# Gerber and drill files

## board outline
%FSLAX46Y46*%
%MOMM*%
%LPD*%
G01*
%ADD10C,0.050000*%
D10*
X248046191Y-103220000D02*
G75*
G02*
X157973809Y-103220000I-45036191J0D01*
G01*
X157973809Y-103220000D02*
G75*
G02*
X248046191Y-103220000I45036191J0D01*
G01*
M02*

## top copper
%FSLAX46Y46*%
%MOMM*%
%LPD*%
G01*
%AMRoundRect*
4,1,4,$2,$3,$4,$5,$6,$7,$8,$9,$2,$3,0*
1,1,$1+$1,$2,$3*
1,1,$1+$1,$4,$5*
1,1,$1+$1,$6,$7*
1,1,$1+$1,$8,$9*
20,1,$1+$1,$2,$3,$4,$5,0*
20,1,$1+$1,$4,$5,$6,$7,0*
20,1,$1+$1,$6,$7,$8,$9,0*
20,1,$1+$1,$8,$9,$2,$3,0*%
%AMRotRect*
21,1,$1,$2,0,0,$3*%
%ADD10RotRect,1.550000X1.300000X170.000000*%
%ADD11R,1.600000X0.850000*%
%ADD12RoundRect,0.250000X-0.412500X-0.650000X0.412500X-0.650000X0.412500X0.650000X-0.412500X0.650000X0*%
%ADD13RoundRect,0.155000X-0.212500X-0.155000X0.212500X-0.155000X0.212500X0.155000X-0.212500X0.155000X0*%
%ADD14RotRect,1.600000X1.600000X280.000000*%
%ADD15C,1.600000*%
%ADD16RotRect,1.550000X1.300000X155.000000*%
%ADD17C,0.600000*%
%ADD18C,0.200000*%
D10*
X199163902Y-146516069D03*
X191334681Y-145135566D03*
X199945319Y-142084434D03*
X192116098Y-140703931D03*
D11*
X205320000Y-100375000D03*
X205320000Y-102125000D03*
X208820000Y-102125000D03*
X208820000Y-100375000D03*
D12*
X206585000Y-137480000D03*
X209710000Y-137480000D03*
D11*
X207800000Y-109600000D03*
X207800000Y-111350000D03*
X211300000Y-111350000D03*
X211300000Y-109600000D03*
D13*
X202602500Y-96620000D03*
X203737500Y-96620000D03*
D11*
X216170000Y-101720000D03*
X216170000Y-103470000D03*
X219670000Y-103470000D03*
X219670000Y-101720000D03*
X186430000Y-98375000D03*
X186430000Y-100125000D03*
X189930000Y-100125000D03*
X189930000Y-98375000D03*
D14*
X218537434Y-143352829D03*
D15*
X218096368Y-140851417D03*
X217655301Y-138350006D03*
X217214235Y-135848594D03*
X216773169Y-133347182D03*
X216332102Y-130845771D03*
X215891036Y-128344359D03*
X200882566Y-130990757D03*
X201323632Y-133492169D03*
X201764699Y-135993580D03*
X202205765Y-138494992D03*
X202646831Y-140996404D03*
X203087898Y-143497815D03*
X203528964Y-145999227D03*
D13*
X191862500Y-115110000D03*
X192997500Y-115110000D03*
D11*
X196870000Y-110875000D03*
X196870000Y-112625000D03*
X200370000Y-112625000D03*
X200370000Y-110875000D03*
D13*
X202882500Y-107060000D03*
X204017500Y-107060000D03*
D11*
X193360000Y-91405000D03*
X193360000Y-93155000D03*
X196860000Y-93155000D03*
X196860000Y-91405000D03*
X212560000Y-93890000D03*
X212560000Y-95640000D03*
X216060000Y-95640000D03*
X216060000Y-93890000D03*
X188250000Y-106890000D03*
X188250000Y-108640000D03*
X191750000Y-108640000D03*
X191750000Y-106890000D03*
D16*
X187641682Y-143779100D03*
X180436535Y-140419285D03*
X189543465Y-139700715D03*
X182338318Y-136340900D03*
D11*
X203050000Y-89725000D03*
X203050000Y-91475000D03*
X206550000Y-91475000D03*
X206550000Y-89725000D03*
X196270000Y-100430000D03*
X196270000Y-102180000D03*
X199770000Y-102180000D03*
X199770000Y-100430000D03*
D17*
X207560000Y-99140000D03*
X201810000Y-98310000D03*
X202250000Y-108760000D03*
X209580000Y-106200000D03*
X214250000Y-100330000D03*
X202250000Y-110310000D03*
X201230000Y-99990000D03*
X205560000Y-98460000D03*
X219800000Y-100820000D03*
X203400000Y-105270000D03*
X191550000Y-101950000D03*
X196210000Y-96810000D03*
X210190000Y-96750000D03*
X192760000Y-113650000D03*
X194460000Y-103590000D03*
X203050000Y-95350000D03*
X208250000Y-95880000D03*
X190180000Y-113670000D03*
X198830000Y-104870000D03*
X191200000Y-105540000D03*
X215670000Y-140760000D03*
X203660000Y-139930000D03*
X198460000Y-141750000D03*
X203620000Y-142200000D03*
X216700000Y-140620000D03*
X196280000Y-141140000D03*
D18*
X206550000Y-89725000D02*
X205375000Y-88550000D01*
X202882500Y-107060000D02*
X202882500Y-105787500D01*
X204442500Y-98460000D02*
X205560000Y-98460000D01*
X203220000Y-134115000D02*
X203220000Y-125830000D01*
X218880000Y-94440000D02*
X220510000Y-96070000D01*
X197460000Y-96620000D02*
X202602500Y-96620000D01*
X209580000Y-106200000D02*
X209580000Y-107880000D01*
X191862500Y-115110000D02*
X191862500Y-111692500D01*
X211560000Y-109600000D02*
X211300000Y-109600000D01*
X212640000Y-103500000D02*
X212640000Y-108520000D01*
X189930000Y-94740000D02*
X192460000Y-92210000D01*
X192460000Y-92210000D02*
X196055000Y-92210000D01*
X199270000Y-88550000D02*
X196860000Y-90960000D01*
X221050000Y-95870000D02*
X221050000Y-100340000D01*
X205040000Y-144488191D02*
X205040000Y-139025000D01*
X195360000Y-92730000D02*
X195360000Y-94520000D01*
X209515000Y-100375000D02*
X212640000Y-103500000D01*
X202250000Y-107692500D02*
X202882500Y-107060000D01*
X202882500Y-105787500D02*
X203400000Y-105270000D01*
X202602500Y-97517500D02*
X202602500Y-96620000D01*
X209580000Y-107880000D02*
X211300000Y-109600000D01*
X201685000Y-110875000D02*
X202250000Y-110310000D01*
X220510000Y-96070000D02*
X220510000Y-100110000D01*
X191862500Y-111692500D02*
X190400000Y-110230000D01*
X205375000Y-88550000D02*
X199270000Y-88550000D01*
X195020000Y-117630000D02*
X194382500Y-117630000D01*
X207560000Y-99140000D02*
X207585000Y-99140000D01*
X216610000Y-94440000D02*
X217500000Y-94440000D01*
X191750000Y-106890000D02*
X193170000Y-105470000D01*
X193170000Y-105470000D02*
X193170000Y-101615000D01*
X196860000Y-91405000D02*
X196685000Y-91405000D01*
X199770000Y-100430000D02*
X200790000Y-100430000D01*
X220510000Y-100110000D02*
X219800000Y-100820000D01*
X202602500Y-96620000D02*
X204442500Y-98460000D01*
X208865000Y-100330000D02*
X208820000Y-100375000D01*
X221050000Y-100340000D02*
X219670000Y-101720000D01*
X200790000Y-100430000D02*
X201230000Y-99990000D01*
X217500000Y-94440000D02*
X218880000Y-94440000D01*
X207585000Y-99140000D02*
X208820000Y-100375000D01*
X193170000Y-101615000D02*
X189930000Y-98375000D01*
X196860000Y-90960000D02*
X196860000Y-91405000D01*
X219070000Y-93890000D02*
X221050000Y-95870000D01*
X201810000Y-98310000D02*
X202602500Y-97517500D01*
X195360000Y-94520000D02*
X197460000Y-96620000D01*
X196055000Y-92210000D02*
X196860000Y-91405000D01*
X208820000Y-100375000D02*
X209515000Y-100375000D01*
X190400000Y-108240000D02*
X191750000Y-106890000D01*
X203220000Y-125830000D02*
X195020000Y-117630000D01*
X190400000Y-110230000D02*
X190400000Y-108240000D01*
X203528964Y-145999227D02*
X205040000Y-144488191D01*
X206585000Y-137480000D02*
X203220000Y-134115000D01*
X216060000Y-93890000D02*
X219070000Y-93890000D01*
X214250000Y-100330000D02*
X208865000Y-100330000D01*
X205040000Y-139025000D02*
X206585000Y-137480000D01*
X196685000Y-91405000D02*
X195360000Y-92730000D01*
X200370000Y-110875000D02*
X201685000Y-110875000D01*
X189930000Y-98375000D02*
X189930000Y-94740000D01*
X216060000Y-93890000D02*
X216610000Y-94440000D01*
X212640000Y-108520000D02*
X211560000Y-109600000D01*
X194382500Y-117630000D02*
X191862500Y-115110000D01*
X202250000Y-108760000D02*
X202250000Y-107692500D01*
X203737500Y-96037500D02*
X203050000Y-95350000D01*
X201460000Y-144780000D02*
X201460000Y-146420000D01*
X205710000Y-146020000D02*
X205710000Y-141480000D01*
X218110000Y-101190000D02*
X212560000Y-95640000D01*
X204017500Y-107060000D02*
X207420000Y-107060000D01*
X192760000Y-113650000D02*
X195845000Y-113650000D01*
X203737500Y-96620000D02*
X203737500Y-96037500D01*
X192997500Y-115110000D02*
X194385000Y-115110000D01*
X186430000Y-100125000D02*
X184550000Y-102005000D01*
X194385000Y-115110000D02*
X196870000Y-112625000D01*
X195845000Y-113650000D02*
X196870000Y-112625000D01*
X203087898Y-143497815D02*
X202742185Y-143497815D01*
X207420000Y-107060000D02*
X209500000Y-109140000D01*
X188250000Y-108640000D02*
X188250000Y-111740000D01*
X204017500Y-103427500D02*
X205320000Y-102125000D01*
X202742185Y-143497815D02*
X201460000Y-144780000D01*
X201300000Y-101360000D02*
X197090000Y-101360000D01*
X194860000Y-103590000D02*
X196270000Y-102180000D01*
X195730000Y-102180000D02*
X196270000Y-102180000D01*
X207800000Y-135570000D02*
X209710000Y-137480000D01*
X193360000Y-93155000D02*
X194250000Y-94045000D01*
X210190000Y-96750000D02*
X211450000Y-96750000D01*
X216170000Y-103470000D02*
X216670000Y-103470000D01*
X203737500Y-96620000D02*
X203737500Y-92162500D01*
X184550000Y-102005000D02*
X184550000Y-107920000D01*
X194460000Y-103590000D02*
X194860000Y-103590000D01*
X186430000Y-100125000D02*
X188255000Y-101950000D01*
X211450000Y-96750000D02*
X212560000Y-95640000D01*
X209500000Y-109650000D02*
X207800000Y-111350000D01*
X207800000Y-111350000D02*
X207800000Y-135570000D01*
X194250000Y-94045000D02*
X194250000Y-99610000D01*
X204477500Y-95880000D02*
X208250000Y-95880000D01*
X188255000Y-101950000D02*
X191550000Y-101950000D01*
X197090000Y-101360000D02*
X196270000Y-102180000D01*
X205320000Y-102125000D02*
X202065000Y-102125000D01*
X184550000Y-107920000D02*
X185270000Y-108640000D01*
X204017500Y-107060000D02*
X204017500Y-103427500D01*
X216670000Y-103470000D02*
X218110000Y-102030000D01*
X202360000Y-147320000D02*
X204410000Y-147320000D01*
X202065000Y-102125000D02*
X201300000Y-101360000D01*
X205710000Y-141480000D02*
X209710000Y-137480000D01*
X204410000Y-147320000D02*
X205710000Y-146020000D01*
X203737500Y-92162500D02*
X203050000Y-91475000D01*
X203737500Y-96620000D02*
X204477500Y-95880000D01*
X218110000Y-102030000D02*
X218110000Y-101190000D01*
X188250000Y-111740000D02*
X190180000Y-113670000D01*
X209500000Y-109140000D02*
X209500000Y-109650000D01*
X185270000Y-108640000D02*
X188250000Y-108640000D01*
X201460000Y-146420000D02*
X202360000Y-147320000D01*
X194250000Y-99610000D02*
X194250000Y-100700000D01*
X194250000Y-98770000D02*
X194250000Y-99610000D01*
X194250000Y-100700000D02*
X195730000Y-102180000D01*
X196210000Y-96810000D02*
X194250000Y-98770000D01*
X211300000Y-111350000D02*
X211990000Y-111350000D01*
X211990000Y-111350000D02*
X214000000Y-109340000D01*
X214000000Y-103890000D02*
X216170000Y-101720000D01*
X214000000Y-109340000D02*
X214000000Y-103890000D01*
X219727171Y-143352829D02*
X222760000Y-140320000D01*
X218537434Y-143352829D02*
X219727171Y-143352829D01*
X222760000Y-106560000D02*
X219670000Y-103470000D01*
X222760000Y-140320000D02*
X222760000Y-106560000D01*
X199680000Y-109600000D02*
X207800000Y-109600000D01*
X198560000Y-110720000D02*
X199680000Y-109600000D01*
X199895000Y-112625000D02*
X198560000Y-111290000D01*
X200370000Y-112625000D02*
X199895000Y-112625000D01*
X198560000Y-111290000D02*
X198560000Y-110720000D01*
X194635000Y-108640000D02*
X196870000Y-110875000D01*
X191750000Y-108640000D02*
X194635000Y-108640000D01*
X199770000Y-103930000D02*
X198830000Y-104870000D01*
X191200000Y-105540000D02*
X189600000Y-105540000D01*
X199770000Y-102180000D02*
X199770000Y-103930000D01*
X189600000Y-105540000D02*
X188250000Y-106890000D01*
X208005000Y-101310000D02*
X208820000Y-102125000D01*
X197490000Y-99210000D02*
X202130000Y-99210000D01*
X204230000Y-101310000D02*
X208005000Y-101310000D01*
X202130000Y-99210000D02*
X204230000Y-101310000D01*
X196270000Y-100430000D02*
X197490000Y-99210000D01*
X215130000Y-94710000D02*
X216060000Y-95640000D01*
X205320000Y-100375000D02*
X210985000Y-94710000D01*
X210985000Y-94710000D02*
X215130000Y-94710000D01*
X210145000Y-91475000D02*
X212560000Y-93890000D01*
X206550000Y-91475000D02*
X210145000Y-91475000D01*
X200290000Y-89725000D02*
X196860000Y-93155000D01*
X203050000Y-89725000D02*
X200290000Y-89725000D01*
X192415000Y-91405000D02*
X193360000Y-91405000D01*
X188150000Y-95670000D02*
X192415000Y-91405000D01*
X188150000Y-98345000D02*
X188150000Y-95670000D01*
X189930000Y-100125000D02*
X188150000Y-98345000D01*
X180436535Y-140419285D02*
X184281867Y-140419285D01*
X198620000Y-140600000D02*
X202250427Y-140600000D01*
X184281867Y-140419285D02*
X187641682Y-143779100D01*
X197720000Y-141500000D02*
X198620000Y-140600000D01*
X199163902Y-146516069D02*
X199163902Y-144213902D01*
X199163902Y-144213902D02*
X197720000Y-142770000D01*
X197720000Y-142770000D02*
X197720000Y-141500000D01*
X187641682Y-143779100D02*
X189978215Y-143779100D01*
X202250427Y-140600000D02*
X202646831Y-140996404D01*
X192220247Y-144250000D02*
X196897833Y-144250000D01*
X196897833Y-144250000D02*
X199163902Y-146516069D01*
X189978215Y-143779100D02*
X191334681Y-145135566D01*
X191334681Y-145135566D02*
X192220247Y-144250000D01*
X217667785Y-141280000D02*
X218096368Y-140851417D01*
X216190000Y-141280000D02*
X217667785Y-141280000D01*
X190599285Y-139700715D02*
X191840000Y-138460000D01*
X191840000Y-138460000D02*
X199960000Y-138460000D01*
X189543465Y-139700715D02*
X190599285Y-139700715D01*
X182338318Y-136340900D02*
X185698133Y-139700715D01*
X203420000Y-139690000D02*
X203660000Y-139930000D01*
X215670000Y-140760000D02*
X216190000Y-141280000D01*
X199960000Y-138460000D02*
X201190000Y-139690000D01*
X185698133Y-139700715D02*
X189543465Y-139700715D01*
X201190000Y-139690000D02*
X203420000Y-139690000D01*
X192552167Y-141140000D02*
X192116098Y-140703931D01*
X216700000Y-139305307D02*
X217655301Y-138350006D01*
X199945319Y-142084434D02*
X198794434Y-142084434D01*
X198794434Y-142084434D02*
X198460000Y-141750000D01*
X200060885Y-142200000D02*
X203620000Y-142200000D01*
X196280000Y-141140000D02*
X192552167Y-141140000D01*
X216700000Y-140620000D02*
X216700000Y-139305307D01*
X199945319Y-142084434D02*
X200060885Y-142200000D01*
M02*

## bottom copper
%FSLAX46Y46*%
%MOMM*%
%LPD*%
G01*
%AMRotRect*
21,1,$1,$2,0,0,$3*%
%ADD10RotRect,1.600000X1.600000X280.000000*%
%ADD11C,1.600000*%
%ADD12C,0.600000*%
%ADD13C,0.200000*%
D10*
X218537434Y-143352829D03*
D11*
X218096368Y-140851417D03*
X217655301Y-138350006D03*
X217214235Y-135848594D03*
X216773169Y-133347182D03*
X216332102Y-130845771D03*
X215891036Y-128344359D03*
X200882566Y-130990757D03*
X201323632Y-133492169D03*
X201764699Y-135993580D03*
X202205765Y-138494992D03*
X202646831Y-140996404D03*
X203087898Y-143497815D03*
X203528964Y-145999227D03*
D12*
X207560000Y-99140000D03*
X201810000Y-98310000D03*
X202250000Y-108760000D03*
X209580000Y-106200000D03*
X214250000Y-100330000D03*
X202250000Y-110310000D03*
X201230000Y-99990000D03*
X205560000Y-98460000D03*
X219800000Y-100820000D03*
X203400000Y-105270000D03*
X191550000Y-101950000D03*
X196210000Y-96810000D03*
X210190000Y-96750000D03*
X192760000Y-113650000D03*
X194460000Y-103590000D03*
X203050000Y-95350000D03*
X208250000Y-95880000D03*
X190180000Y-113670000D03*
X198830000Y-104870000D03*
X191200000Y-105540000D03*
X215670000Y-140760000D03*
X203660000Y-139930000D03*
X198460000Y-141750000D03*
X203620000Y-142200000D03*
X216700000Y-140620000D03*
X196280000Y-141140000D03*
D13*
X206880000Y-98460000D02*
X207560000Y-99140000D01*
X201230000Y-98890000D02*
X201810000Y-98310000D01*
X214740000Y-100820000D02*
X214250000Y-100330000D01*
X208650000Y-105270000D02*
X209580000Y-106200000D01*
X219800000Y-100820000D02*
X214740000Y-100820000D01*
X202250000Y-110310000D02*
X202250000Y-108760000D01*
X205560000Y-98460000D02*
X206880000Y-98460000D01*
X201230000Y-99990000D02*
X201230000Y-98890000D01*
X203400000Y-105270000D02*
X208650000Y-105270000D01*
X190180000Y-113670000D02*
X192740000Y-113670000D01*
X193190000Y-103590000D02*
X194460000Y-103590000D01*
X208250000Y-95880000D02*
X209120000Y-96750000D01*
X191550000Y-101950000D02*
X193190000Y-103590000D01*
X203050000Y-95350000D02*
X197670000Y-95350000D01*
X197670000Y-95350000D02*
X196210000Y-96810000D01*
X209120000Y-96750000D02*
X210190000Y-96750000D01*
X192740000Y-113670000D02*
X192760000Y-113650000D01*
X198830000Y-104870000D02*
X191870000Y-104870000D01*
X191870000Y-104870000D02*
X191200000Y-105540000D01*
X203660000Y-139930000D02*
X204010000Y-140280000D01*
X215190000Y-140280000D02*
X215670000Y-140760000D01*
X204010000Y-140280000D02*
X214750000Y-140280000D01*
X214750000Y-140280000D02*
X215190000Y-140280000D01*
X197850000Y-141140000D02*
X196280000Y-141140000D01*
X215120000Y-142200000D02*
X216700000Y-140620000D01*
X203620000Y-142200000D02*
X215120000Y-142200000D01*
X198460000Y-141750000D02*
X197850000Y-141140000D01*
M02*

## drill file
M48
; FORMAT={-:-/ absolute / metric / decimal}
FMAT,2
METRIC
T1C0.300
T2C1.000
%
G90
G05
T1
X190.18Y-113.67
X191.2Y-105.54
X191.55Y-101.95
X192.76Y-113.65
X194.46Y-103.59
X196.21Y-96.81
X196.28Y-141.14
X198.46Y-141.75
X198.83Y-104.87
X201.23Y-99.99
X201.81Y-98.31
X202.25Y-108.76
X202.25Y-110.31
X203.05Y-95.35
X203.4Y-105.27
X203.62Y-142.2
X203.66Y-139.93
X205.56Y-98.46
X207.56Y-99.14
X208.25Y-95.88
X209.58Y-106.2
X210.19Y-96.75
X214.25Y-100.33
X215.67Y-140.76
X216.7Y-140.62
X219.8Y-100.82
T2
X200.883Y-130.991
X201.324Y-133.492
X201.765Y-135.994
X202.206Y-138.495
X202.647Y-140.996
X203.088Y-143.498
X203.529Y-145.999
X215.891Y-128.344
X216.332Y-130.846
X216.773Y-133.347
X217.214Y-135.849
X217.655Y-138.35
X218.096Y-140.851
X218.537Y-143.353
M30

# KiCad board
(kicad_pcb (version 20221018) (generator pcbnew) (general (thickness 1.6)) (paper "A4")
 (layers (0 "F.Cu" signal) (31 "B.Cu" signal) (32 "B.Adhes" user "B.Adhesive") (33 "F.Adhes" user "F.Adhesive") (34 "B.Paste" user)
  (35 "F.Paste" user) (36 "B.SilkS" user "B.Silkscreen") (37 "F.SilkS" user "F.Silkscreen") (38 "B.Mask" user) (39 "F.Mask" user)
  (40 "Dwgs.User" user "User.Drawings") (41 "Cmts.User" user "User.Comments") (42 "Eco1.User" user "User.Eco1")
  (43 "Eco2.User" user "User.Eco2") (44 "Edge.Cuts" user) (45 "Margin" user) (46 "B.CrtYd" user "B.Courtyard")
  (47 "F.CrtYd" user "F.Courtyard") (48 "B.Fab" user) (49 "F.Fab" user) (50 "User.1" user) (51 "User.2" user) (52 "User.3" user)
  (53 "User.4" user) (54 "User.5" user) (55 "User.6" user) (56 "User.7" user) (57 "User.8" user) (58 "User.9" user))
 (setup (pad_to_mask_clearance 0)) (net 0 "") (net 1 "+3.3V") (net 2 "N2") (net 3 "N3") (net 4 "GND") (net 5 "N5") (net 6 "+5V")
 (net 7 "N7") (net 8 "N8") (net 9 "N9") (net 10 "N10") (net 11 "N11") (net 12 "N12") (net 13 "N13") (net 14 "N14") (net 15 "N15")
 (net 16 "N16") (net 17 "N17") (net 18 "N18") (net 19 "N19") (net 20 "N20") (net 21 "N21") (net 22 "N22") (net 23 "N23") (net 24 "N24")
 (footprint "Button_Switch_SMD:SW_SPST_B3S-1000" (layer "F.Cu") (at 195.64 143.61 170)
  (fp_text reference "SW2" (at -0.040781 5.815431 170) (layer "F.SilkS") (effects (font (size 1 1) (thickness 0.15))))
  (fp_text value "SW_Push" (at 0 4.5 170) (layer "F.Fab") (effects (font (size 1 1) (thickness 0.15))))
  (pad "1" smd rect (at -3.975 -2.25 170) (size 1.55 1.3) (layers "F.Cu" "F.Paste" "F.Mask") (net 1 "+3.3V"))
  (pad "1" smd rect (at 3.975 -2.25 170) (size 1.55 1.3) (layers "F.Cu" "F.Paste" "F.Mask") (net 1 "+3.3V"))
  (pad "2" smd rect (at -3.975 2.25 170) (size 1.55 1.3) (layers "F.Cu" "F.Paste" "F.Mask") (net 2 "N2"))
  (pad "2" smd rect (at 3.975 2.25 170) (size 1.55 1.3) (layers "F.Cu" "F.Paste" "F.Mask") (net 2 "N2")))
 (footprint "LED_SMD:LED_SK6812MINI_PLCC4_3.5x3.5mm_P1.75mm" (layer "F.Cu") (at 207.07 101.25)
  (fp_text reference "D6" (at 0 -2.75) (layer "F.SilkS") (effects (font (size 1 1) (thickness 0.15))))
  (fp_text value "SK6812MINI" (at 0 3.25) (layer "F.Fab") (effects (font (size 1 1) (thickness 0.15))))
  (pad "1" smd rect (at -1.75 -0.875) (size 1.6 0.85) (layers "F.Cu" "F.Paste" "F.Mask") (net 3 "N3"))
  (pad "2" smd rect (at -1.75 0.875) (size 1.6 0.85) (layers "F.Cu" "F.Paste" "F.Mask") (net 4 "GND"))
  (pad "3" smd rect (at 1.75 0.875) (size 1.6 0.85) (layers "F.Cu" "F.Paste" "F.Mask") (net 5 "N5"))
  (pad "4" smd rect (at 1.75 -0.875) (size 1.6 0.85) (layers "F.Cu" "F.Paste" "F.Mask") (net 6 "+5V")))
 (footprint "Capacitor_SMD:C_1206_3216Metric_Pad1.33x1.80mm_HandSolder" (layer "F.Cu") (at 208.1475 137.48)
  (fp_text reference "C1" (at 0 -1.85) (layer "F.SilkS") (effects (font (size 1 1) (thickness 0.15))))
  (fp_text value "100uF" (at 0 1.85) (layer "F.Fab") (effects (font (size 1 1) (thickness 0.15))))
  (pad "1" smd roundrect (at -1.5625 0) (size 1.325 1.8) (layers "F.Cu" "F.Paste" "F.Mask") (roundrect_rratio 0.1886792453) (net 6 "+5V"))
  (pad "2" smd roundrect (at 1.5625 0) (size 1.325 1.8) (layers "F.Cu" "F.Paste" "F.Mask") (roundrect_rratio 0.1886792453) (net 4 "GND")))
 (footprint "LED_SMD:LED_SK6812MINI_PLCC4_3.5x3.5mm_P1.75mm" (layer "F.Cu") (at 209.55 110.475)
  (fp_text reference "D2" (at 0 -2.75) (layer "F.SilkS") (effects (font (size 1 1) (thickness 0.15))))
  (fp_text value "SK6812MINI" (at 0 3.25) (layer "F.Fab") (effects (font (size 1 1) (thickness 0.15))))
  (pad "1" smd rect (at -1.75 -0.875) (size 1.6 0.85) (layers "F.Cu" "F.Paste" "F.Mask") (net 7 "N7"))
  (pad "2" smd rect (at -1.75 0.875) (size 1.6 0.85) (layers "F.Cu" "F.Paste" "F.Mask") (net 4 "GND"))
  (pad "3" smd rect (at 1.75 0.875) (size 1.6 0.85) (layers "F.Cu" "F.Paste" "F.Mask") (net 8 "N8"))
  (pad "4" smd rect (at 1.75 -0.875) (size 1.6 0.85) (layers "F.Cu" "F.Paste" "F.Mask") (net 6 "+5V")))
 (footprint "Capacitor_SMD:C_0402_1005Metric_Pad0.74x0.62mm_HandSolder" (layer "F.Cu") (at 203.17 96.62)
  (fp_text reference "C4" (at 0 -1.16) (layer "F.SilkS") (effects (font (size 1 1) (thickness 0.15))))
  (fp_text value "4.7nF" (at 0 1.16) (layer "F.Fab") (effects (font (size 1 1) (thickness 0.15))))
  (pad "1" smd roundrect (at -0.5675 0) (size 0.735 0.62) (layers "F.Cu" "F.Paste" "F.Mask") (roundrect_rratio 0.25) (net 6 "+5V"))
  (pad "2" smd roundrect (at 0.5675 0) (size 0.735 0.62) (layers "F.Cu" "F.Paste" "F.Mask") (roundrect_rratio 0.25) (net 4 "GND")))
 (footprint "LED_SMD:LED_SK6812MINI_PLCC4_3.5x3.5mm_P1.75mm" (layer "F.Cu") (at 217.92 102.595)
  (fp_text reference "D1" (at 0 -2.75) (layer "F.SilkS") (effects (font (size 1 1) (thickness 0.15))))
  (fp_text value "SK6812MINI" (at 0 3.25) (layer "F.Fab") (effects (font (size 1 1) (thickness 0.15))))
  (pad "1" smd rect (at -1.75 -0.875) (size 1.6 0.85) (layers "F.Cu" "F.Paste" "F.Mask") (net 8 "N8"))
  (pad "2" smd rect (at -1.75 0.875) (size 1.6 0.85) (layers "F.Cu" "F.Paste" "F.Mask") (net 4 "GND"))
  (pad "3" smd rect (at 1.75 0.875) (size 1.6 0.85) (layers "F.Cu" "F.Paste" "F.Mask") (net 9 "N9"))
  (pad "4" smd rect (at 1.75 -0.875) (size 1.6 0.85) (layers "F.Cu" "F.Paste" "F.Mask") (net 6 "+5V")))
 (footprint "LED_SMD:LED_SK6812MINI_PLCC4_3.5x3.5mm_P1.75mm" (layer "F.Cu") (at 188.18 99.25)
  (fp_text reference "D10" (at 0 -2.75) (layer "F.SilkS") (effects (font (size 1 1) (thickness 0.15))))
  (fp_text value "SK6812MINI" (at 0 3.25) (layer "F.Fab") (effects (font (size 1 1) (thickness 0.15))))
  (pad "1" smd rect (at -1.75 -0.875) (size 1.6 0.85) (layers "F.Cu" "F.Paste" "F.Mask") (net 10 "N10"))
  (pad "2" smd rect (at -1.75 0.875) (size 1.6 0.85) (layers "F.Cu" "F.Paste" "F.Mask") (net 4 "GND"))
  (pad "3" smd rect (at 1.75 0.875) (size 1.6 0.85) (layers "F.Cu" "F.Paste" "F.Mask") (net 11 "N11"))
  (pad "4" smd rect (at 1.75 -0.875) (size 1.6 0.85) (layers "F.Cu" "F.Paste" "F.Mask") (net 6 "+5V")))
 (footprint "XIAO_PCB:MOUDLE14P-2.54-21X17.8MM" (layer "F.Cu") (at 209.71 137.171793 -80)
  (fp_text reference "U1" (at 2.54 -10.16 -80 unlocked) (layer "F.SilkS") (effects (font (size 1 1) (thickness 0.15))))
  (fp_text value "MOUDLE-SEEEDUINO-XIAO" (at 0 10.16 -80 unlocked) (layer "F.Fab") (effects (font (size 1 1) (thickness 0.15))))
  (pad "1" thru_hole rect (at 7.62 -7.62 280) (size 1.6 1.6) (drill 1) (layers "*.Cu" "*.Mask") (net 9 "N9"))
  (pad "2" thru_hole circle (at 5.08 -7.62 280) (size 1.6 1.6) (drill 1) (layers "*.Cu" "*.Mask") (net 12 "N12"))
  (pad "3" thru_hole circle (at 2.54 -7.62 280) (size 1.6 1.6) (drill 1) (layers "*.Cu" "*.Mask") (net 2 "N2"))
  (pad "4" thru_hole circle (at 0 -7.62 280) (size 1.6 1.6) (drill 1) (layers "*.Cu" "*.Mask") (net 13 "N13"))
  (pad "5" thru_hole circle (at -2.54 -7.62 280) (size 1.6 1.6) (drill 1) (layers "*.Cu" "*.Mask") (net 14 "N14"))
  (pad "6" thru_hole circle (at -5.08 -7.62 280) (size 1.6 1.6) (drill 1) (layers "*.Cu" "*.Mask") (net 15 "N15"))
  (pad "7" thru_hole circle (at -7.62 -7.62 280) (size 1.6 1.6) (drill 1) (layers "*.Cu" "*.Mask") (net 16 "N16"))
  (pad "8" thru_hole circle (at -7.62 7.62 280) (size 1.6 1.6) (drill 1) (layers "*.Cu" "*.Mask") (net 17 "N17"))
  (pad "9" thru_hole circle (at -5.08 7.62 280) (size 1.6 1.6) (drill 1) (layers "*.Cu" "*.Mask") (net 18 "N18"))
  (pad "10" thru_hole circle (at -2.54 7.62 280) (size 1.6 1.6) (drill 1) (layers "*.Cu" "*.Mask") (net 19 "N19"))
  (pad "11" thru_hole circle (at 0 7.62 280) (size 1.6 1.6) (drill 1) (layers "*.Cu" "*.Mask") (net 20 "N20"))
  (pad "12" thru_hole circle (at 2.54 7.62 280) (size 1.6 1.6) (drill 1) (layers "*.Cu" "*.Mask") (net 1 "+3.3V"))
  (pad "13" thru_hole circle (at 5.08 7.62 280) (size 1.6 1.6) (drill 1) (layers "*.Cu" "*.Mask") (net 4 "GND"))
  (pad "14" thru_hole circle (at 7.62 7.62 280) (size 1.6 1.6) (drill 1) (layers "*.Cu" "*.Mask") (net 6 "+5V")))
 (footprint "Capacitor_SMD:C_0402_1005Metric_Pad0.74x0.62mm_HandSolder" (layer "F.Cu") (at 192.43 115.11)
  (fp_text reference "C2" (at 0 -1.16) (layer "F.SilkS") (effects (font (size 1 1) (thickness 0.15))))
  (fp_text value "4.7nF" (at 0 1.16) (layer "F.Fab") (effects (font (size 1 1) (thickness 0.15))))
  (pad "1" smd roundrect (at -0.5675 0) (size 0.735 0.62) (layers "F.Cu" "F.Paste" "F.Mask") (roundrect_rratio 0.25) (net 6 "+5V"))
  (pad "2" smd roundrect (at 0.5675 0) (size 0.735 0.62) (layers "F.Cu" "F.Paste" "F.Mask") (roundrect_rratio 0.25) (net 4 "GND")))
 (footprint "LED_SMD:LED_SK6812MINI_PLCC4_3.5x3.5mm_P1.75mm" (layer "F.Cu") (at 198.62 111.75)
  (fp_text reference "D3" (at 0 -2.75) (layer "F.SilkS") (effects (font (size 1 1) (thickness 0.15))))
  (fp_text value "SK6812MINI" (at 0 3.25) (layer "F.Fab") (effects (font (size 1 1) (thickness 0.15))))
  (pad "1" smd rect (at -1.75 -0.875) (size 1.6 0.85) (layers "F.Cu" "F.Paste" "F.Mask") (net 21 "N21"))
  (pad "2" smd rect (at -1.75 0.875) (size 1.6 0.85) (layers "F.Cu" "F.Paste" "F.Mask") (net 4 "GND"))
  (pad "3" smd rect (at 1.75 0.875) (size 1.6 0.85) (layers "F.Cu" "F.Paste" "F.Mask") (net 7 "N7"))
  (pad "4" smd rect (at 1.75 -0.875) (size 1.6 0.85) (layers "F.Cu" "F.Paste" "F.Mask") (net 6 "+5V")))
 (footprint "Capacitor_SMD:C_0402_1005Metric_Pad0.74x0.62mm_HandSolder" (layer "F.Cu") (at 203.45 107.06)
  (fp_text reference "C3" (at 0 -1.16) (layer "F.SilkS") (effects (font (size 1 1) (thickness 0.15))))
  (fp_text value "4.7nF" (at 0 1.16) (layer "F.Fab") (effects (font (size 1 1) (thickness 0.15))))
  (pad "1" smd roundrect (at -0.5675 0) (size 0.735 0.62) (layers "F.Cu" "F.Paste" "F.Mask") (roundrect_rratio 0.25) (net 6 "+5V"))
  (pad "2" smd roundrect (at 0.5675 0) (size 0.735 0.62) (layers "F.Cu" "F.Paste" "F.Mask") (roundrect_rratio 0.25) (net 4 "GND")))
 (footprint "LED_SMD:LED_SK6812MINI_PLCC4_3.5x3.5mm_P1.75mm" (layer "F.Cu") (at 195.11 92.28)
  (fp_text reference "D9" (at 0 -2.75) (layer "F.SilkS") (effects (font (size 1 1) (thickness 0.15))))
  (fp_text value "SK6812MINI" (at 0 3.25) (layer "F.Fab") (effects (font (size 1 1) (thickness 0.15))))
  (pad "1" smd rect (at -1.75 -0.875) (size 1.6 0.85) (layers "F.Cu" "F.Paste" "F.Mask") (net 11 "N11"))
  (pad "2" smd rect (at -1.75 0.875) (size 1.6 0.85) (layers "F.Cu" "F.Paste" "F.Mask") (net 4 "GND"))
  (pad "3" smd rect (at 1.75 0.875) (size 1.6 0.85) (layers "F.Cu" "F.Paste" "F.Mask") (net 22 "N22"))
  (pad "4" smd rect (at 1.75 -0.875) (size 1.6 0.85) (layers "F.Cu" "F.Paste" "F.Mask") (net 6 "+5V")))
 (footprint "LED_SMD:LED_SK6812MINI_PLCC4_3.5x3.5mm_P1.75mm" (layer "F.Cu") (at 214.31 94.765)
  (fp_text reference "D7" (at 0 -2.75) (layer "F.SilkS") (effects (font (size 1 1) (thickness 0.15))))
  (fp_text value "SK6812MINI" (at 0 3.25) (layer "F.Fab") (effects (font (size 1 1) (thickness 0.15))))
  (pad "1" smd rect (at -1.75 -0.875) (size 1.6 0.85) (layers "F.Cu" "F.Paste" "F.Mask") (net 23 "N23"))
  (pad "2" smd rect (at -1.75 0.875) (size 1.6 0.85) (layers "F.Cu" "F.Paste" "F.Mask") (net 4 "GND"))
  (pad "3" smd rect (at 1.75 0.875) (size 1.6 0.85) (layers "F.Cu" "F.Paste" "F.Mask") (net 3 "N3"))
  (pad "4" smd rect (at 1.75 -0.875) (size 1.6 0.85) (layers "F.Cu" "F.Paste" "F.Mask") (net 6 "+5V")))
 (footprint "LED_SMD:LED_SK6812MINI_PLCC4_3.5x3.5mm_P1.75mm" (layer "F.Cu") (at 190 107.765)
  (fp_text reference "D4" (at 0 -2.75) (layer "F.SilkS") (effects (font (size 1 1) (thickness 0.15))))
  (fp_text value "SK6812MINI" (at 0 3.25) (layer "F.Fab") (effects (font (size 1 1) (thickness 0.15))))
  (pad "1" smd rect (at -1.75 -0.875) (size 1.6 0.85) (layers "F.Cu" "F.Paste" "F.Mask") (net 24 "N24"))
  (pad "2" smd rect (at -1.75 0.875) (size 1.6 0.85) (layers "F.Cu" "F.Paste" "F.Mask") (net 4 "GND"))
  (pad "3" smd rect (at 1.75 0.875) (size 1.6 0.85) (layers "F.Cu" "F.Paste" "F.Mask") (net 21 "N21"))
  (pad "4" smd rect (at 1.75 -0.875) (size 1.6 0.85) (layers "F.Cu" "F.Paste" "F.Mask") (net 6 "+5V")))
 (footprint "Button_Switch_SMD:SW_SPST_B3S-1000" (layer "F.Cu") (at 184.99 140.06 155)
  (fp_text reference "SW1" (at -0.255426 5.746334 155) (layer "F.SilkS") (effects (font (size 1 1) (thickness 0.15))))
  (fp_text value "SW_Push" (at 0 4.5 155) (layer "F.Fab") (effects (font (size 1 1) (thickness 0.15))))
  (pad "1" smd rect (at -3.975 -2.25 155) (size 1.55 1.3) (layers "F.Cu" "F.Paste" "F.Mask") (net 1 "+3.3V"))
  (pad "1" smd rect (at 3.975 -2.25 155) (size 1.55 1.3) (layers "F.Cu" "F.Paste" "F.Mask") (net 1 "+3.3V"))
  (pad "2" smd rect (at -3.975 2.25 155) (size 1.55 1.3) (layers "F.Cu" "F.Paste" "F.Mask") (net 12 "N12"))
  (pad "2" smd rect (at 3.975 2.25 155) (size 1.55 1.3) (layers "F.Cu" "F.Paste" "F.Mask") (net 12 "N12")))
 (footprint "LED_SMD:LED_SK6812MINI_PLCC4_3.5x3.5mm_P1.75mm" (layer "F.Cu") (at 204.8 90.6)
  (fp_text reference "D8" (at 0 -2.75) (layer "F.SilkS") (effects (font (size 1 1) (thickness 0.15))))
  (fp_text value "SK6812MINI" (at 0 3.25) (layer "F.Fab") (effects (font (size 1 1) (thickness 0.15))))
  (pad "1" smd rect (at -1.75 -0.875) (size 1.6 0.85) (layers "F.Cu" "F.Paste" "F.Mask") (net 22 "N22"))
  (pad "2" smd rect (at -1.75 0.875) (size 1.6 0.85) (layers "F.Cu" "F.Paste" "F.Mask") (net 4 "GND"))
  (pad "3" smd rect (at 1.75 0.875) (size 1.6 0.85) (layers "F.Cu" "F.Paste" "F.Mask") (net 23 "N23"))
  (pad "4" smd rect (at 1.75 -0.875) (size 1.6 0.85) (layers "F.Cu" "F.Paste" "F.Mask") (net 6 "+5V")))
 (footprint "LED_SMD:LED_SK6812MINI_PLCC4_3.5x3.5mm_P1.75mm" (layer "F.Cu") (at 198.02 101.305)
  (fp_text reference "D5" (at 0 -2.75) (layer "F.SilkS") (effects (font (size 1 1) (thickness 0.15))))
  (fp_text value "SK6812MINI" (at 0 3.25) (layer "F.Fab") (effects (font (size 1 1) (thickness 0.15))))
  (pad "1" smd rect (at -1.75 -0.875) (size 1.6 0.85) (layers "F.Cu" "F.Paste" "F.Mask") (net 5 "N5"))
  (pad "2" smd rect (at -1.75 0.875) (size 1.6 0.85) (layers "F.Cu" "F.Paste" "F.Mask") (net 4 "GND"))
  (pad "3" smd rect (at 1.75 0.875) (size 1.6 0.85) (layers "F.Cu" "F.Paste" "F.Mask") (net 24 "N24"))
  (pad "4" smd rect (at 1.75 -0.875) (size 1.6 0.85) (layers "F.Cu" "F.Paste" "F.Mask") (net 6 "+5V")))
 (gr_circle (center 203.01 103.22) (end 227.92 140.74) (stroke (width 0.05) (type default)) (fill none) (layer "Edge.Cuts"))
 (segment (start 206.55 89.725) (end 205.375 88.55) (width 0.2) (layer "F.Cu") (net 6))
 (segment (start 202.8825 107.06) (end 202.8825 105.7875) (width 0.2) (layer "F.Cu") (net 6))
 (segment (start 204.4425 98.46) (end 205.56 98.46) (width 0.2) (layer "F.Cu") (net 6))
 (segment (start 203.22 134.115) (end 203.22 125.83) (width 0.2) (layer "F.Cu") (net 6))
 (segment (start 218.88 94.44) (end 220.51 96.07) (width 0.2) (layer "F.Cu") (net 6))
 (segment (start 197.46 96.62) (end 202.6025 96.62) (width 0.2) (layer "F.Cu") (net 6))
 (segment (start 209.58 106.2) (end 209.58 107.88) (width 0.2) (layer "F.Cu") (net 6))
 (segment (start 191.8625 115.11) (end 191.8625 111.6925) (width 0.2) (layer "F.Cu") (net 6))
 (segment (start 211.56 109.6) (end 211.3 109.6) (width 0.2) (layer "F.Cu") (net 6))
 (segment (start 212.64 103.5) (end 212.64 108.52) (width 0.2) (layer "F.Cu") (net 6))
 (segment (start 189.93 94.74) (end 192.46 92.21) (width 0.2) (layer "F.Cu") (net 6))
 (segment (start 192.46 92.21) (end 196.055 92.21) (width 0.2) (layer "F.Cu") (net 6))
 (segment (start 199.27 88.55) (end 196.86 90.96) (width 0.2) (layer "F.Cu") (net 6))
 (segment (start 221.05 95.87) (end 221.05 100.34) (width 0.2) (layer "F.Cu") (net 6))
 (segment (start 205.04 144.488191) (end 205.04 139.025) (width 0.2) (layer "F.Cu") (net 6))
 (segment (start 195.36 92.73) (end 195.36 94.52) (width 0.2) (layer "F.Cu") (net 6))
 (segment (start 209.515 100.375) (end 212.64 103.5) (width 0.2) (layer "F.Cu") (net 6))
 (segment (start 202.25 107.6925) (end 202.8825 107.06) (width 0.2) (layer "F.Cu") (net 6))
 (segment (start 202.8825 105.7875) (end 203.4 105.27) (width 0.2) (layer "F.Cu") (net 6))
 (segment (start 202.6025 97.5175) (end 202.6025 96.62) (width 0.2) (layer "F.Cu") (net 6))
 (segment (start 209.58 107.88) (end 211.3 109.6) (width 0.2) (layer "F.Cu") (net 6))
 (segment (start 201.685 110.875) (end 202.25 110.31) (width 0.2) (layer "F.Cu") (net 6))
 (segment (start 220.51 96.07) (end 220.51 100.11) (width 0.2) (layer "F.Cu") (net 6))
 (segment (start 191.8625 111.6925) (end 190.4 110.23) (width 0.2) (layer "F.Cu") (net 6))
 (segment (start 205.375 88.55) (end 199.27 88.55) (width 0.2) (layer "F.Cu") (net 6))
 (segment (start 195.02 117.63) (end 194.3825 117.63) (width 0.2) (layer "F.Cu") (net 6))
 (segment (start 207.56 99.14) (end 207.585 99.14) (width 0.2) (layer "F.Cu") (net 6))
 (segment (start 216.61 94.44) (end 217.5 94.44) (width 0.2) (layer "F.Cu") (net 6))
 (segment (start 191.75 106.89) (end 193.17 105.47) (width 0.2) (layer "F.Cu") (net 6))
 (segment (start 193.17 105.47) (end 193.17 101.615) (width 0.2) (layer "F.Cu") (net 6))
 (segment (start 196.86 91.405) (end 196.685 91.405) (width 0.2) (layer "F.Cu") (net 6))
 (segment (start 199.77 100.43) (end 200.79 100.43) (width 0.2) (layer "F.Cu") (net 6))
 (segment (start 220.51 100.11) (end 219.8 100.82) (width 0.2) (layer "F.Cu") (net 6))
 (segment (start 202.6025 96.62) (end 204.4425 98.46) (width 0.2) (layer "F.Cu") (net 6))
 (segment (start 208.865 100.33) (end 208.82 100.375) (width 0.2) (layer "F.Cu") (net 6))
 (segment (start 221.05 100.34) (end 219.67 101.72) (width 0.2) (layer "F.Cu") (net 6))
 (segment (start 200.79 100.43) (end 201.23 99.99) (width 0.2) (layer "F.Cu") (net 6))
 (segment (start 217.5 94.44) (end 218.88 94.44) (width 0.2) (layer "F.Cu") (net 6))
 (segment (start 207.585 99.14) (end 208.82 100.375) (width 0.2) (layer "F.Cu") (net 6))
 (segment (start 193.17 101.615) (end 189.93 98.375) (width 0.2) (layer "F.Cu") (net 6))
 (segment (start 196.86 90.96) (end 196.86 91.405) (width 0.2) (layer "F.Cu") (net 6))
 (segment (start 219.07 93.89) (end 221.05 95.87) (width 0.2) (layer "F.Cu") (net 6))
 (segment (start 201.81 98.31) (end 202.6025 97.5175) (width 0.2) (layer "F.Cu") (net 6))
 (segment (start 195.36 94.52) (end 197.46 96.62) (width 0.2) (layer "F.Cu") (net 6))
 (segment (start 196.055 92.21) (end 196.86 91.405) (width 0.2) (layer "F.Cu") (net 6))
 (segment (start 208.82 100.375) (end 209.515 100.375) (width 0.2) (layer "F.Cu") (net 6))
 (segment (start 190.4 108.24) (end 191.75 106.89) (width 0.2) (layer "F.Cu") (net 6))
 (segment (start 203.22 125.83) (end 195.02 117.63) (width 0.2) (layer "F.Cu") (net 6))
 (segment (start 190.4 110.23) (end 190.4 108.24) (width 0.2) (layer "F.Cu") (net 6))
 (segment (start 203.528964 145.999227) (end 205.04 144.488191) (width 0.2) (layer "F.Cu") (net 6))
 (segment (start 206.585 137.48) (end 203.22 134.115) (width 0.2) (layer "F.Cu") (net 6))
 (segment (start 216.06 93.89) (end 219.07 93.89) (width 0.2) (layer "F.Cu") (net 6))
 (segment (start 214.25 100.33) (end 208.865 100.33) (width 0.2) (layer "F.Cu") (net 6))
 (segment (start 205.04 139.025) (end 206.585 137.48) (width 0.2) (layer "F.Cu") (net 6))
 (segment (start 196.685 91.405) (end 195.36 92.73) (width 0.2) (layer "F.Cu") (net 6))
 (segment (start 200.37 110.875) (end 201.685 110.875) (width 0.2) (layer "F.Cu") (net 6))
 (segment (start 189.93 98.375) (end 189.93 94.74) (width 0.2) (layer "F.Cu") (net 6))
 (segment (start 216.06 93.89) (end 216.61 94.44) (width 0.2) (layer "F.Cu") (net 6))
 (segment (start 212.64 108.52) (end 211.56 109.6) (width 0.2) (layer "F.Cu") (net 6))
 (segment (start 194.3825 117.63) (end 191.8625 115.11) (width 0.2) (layer "F.Cu") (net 6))
 (segment (start 202.25 108.76) (end 202.25 107.6925) (width 0.2) (layer "F.Cu") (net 6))
 (via (at 207.56 99.14) (size 0.6) (drill 0.3) (layers "F.Cu" "B.Cu") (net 6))
 (via (at 201.81 98.31) (size 0.6) (drill 0.3) (layers "F.Cu" "B.Cu") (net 6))
 (via (at 202.25 108.76) (size 0.6) (drill 0.3) (layers "F.Cu" "B.Cu") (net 6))
 (via (at 209.58 106.2) (size 0.6) (drill 0.3) (layers "F.Cu" "B.Cu") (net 6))
 (via (at 214.25 100.33) (size 0.6) (drill 0.3) (layers "F.Cu" "B.Cu") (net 6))
 (via (at 202.25 110.31) (size 0.6) (drill 0.3) (layers "F.Cu" "B.Cu") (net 6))
 (via (at 201.23 99.99) (size 0.6) (drill 0.3) (layers "F.Cu" "B.Cu") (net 6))
 (via (at 205.56 98.46) (size 0.6) (drill 0.3) (layers "F.Cu" "B.Cu") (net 6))
 (via (at 219.8 100.82) (size 0.6) (drill 0.3) (layers "F.Cu" "B.Cu") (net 6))
 (via (at 203.4 105.27) (size 0.6) (drill 0.3) (layers "F.Cu" "B.Cu") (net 6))
 (segment (start 206.88 98.46) (end 207.56 99.14) (width 0.2) (layer "B.Cu") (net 6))
 (segment (start 201.23 98.89) (end 201.81 98.31) (width 0.2) (layer "B.Cu") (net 6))
 (segment (start 214.74 100.82) (end 214.25 100.33) (width 0.2) (layer "B.Cu") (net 6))
 (segment (start 208.65 105.27) (end 209.58 106.2) (width 0.2) (layer "B.Cu") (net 6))
 (segment (start 219.8 100.82) (end 214.74 100.82) (width 0.2) (layer "B.Cu") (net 6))
 (segment (start 202.25 110.31) (end 202.25 108.76) (width 0.2) (layer "B.Cu") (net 6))
 (segment (start 205.56 98.46) (end 206.88 98.46) (width 0.2) (layer "B.Cu") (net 6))
 (segment (start 201.23 99.99) (end 201.23 98.89) (width 0.2) (layer "B.Cu") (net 6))
 (segment (start 203.4 105.27) (end 208.65 105.27) (width 0.2) (layer "B.Cu") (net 6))
 (segment (start 203.7375 96.0375) (end 203.05 95.35) (width 0.2) (layer "F.Cu") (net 4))
 (segment (start 201.46 144.78) (end 201.46 146.42) (width 0.2) (layer "F.Cu") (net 4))
 (segment (start 205.71 146.02) (end 205.71 141.48) (width 0.2) (layer "F.Cu") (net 4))
 (segment (start 218.11 101.19) (end 212.56 95.64) (width 0.2) (layer "F.Cu") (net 4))
 (segment (start 204.0175 107.06) (end 207.42 107.06) (width 0.2) (layer "F.Cu") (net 4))
 (segment (start 192.76 113.65) (end 195.845 113.65) (width 0.2) (layer "F.Cu") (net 4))
 (segment (start 203.7375 96.62) (end 203.7375 96.0375) (width 0.2) (layer "F.Cu") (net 4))
 (segment (start 192.9975 115.11) (end 194.385 115.11) (width 0.2) (layer "F.Cu") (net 4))
 (segment (start 186.43 100.125) (end 184.55 102.005) (width 0.2) (layer "F.Cu") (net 4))
 (segment (start 194.385 115.11) (end 196.87 112.625) (width 0.2) (layer "F.Cu") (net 4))
 (segment (start 195.845 113.65) (end 196.87 112.625) (width 0.2) (layer "F.Cu") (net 4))
 (segment (start 203.087898 143.497815) (end 202.742185 143.497815) (width 0.2) (layer "F.Cu") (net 4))
 (segment (start 207.42 107.06) (end 209.5 109.14) (width 0.2) (layer "F.Cu") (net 4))
 (segment (start 188.25 108.64) (end 188.25 111.74) (width 0.2) (layer "F.Cu") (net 4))
 (segment (start 204.0175 103.4275) (end 205.32 102.125) (width 0.2) (layer "F.Cu") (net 4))
 (segment (start 202.742185 143.497815) (end 201.46 144.78) (width 0.2) (layer "F.Cu") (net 4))
 (segment (start 201.3 101.36) (end 197.09 101.36) (width 0.2) (layer "F.Cu") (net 4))
 (segment (start 194.86 103.59) (end 196.27 102.18) (width 0.2) (layer "F.Cu") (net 4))
 (segment (start 195.73 102.18) (end 196.27 102.18) (width 0.2) (layer "F.Cu") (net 4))
 (segment (start 207.8 135.57) (end 209.71 137.48) (width 0.2) (layer "F.Cu") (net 4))
 (segment (start 193.36 93.155) (end 194.25 94.045) (width 0.2) (layer "F.Cu") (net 4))
 (segment (start 210.19 96.75) (end 211.45 96.75) (width 0.2) (layer "F.Cu") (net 4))
 (segment (start 216.17 103.47) (end 216.67 103.47) (width 0.2) (layer "F.Cu") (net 4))
 (segment (start 203.7375 96.62) (end 203.7375 92.1625) (width 0.2) (layer "F.Cu") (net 4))
 (segment (start 184.55 102.005) (end 184.55 107.92) (width 0.2) (layer "F.Cu") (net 4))
 (segment (start 194.46 103.59) (end 194.86 103.59) (width 0.2) (layer "F.Cu") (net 4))
 (segment (start 186.43 100.125) (end 188.255 101.95) (width 0.2) (layer "F.Cu") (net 4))
 (segment (start 211.45 96.75) (end 212.56 95.64) (width 0.2) (layer "F.Cu") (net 4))
 (segment (start 209.5 109.65) (end 207.8 111.35) (width 0.2) (layer "F.Cu") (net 4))
 (segment (start 207.8 111.35) (end 207.8 135.57) (width 0.2) (layer "F.Cu") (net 4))
 (segment (start 194.25 94.045) (end 194.25 99.61) (width 0.2) (layer "F.Cu") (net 4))
 (segment (start 204.4775 95.88) (end 208.25 95.88) (width 0.2) (layer "F.Cu") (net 4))
 (segment (start 188.255 101.95) (end 191.55 101.95) (width 0.2) (layer "F.Cu") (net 4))
 (segment (start 197.09 101.36) (end 196.27 102.18) (width 0.2) (layer "F.Cu") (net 4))
 (segment (start 205.32 102.125) (end 202.065 102.125) (width 0.2) (layer "F.Cu") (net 4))
 (segment (start 184.55 107.92) (end 185.27 108.64) (width 0.2) (layer "F.Cu") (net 4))
 (segment (start 204.0175 107.06) (end 204.0175 103.4275) (width 0.2) (layer "F.Cu") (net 4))
 (segment (start 216.67 103.47) (end 218.11 102.03) (width 0.2) (layer "F.Cu") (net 4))
 (segment (start 202.36 147.32) (end 204.41 147.32) (width 0.2) (layer "F.Cu") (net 4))
 (segment (start 202.065 102.125) (end 201.3 101.36) (width 0.2) (layer "F.Cu") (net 4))
 (segment (start 205.71 141.48) (end 209.71 137.48) (width 0.2) (layer "F.Cu") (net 4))
 (segment (start 204.41 147.32) (end 205.71 146.02) (width 0.2) (layer "F.Cu") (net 4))
 (segment (start 203.7375 92.1625) (end 203.05 91.475) (width 0.2) (layer "F.Cu") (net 4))
 (segment (start 203.7375 96.62) (end 204.4775 95.88) (width 0.2) (layer "F.Cu") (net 4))
 (segment (start 218.11 102.03) (end 218.11 101.19) (width 0.2) (layer "F.Cu") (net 4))
 (segment (start 188.25 111.74) (end 190.18 113.67) (width 0.2) (layer "F.Cu") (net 4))
 (segment (start 209.5 109.14) (end 209.5 109.65) (width 0.2) (layer "F.Cu") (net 4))
 (segment (start 185.27 108.64) (end 188.25 108.64) (width 0.2) (layer "F.Cu") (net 4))
 (segment (start 201.46 146.42) (end 202.36 147.32) (width 0.2) (layer "F.Cu") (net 4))
 (segment (start 194.25 99.61) (end 194.25 100.7) (width 0.2) (layer "F.Cu") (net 4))
 (segment (start 194.25 98.77) (end 194.25 99.61) (width 0.2) (layer "F.Cu") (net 4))
 (segment (start 194.25 100.7) (end 195.73 102.18) (width 0.2) (layer "F.Cu") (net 4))
 (segment (start 196.21 96.81) (end 194.25 98.77) (width 0.2) (layer "F.Cu") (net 4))
 (via (at 191.55 101.95) (size 0.6) (drill 0.3) (layers "F.Cu" "B.Cu") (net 4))
 (via (at 196.21 96.81) (size 0.6) (drill 0.3) (layers "F.Cu" "B.Cu") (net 4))
 (via (at 210.19 96.75) (size 0.6) (drill 0.3) (layers "F.Cu" "B.Cu") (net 4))
 (via (at 192.76 113.65) (size 0.6) (drill 0.3) (layers "F.Cu" "B.Cu") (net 4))
 (via (at 194.46 103.59) (size 0.6) (drill 0.3) (layers "F.Cu" "B.Cu") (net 4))
 (via (at 203.05 95.35) (size 0.6) (drill 0.3) (layers "F.Cu" "B.Cu") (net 4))
 (via (at 208.25 95.88) (size 0.6) (drill 0.3) (layers "F.Cu" "B.Cu") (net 4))
 (via (at 190.18 113.67) (size 0.6) (drill 0.3) (layers "F.Cu" "B.Cu") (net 4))
 (segment (start 190.18 113.67) (end 192.74 113.67) (width 0.2) (layer "B.Cu") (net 4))
 (segment (start 193.19 103.59) (end 194.46 103.59) (width 0.2) (layer "B.Cu") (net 4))
 (segment (start 208.25 95.88) (end 209.12 96.75) (width 0.2) (layer "B.Cu") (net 4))
 (segment (start 191.55 101.95) (end 193.19 103.59) (width 0.2) (layer "B.Cu") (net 4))
 (segment (start 203.05 95.35) (end 197.67 95.35) (width 0.2) (layer "B.Cu") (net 4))
 (segment (start 197.67 95.35) (end 196.21 96.81) (width 0.2) (layer "B.Cu") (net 4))
 (segment (start 209.12 96.75) (end 210.19 96.75) (width 0.2) (layer "B.Cu") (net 4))
 (segment (start 192.74 113.67) (end 192.76 113.65) (width 0.2) (layer "B.Cu") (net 4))
 (segment (start 211.3 111.35) (end 211.99 111.35) (width 0.2) (layer "F.Cu") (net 8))
 (segment (start 211.99 111.35) (end 214 109.34) (width 0.2) (layer "F.Cu") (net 8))
 (segment (start 214 103.89) (end 216.17 101.72) (width 0.2) (layer "F.Cu") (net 8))
 (segment (start 214 109.34) (end 214 103.89) (width 0.2) (layer "F.Cu") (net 8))
 (segment (start 219.727171 143.352829) (end 222.76 140.32) (width 0.2) (layer "F.Cu") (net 9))
 (segment (start 218.537434 143.352829) (end 219.727171 143.352829) (width 0.2) (layer "F.Cu") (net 9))
 (segment (start 222.76 106.56) (end 219.67 103.47) (width 0.2) (layer "F.Cu") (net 9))
 (segment (start 222.76 140.32) (end 222.76 106.56) (width 0.2) (layer "F.Cu") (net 9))
 (segment (start 199.68 109.6) (end 207.8 109.6) (width 0.2) (layer "F.Cu") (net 7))
 (segment (start 198.56 110.72) (end 199.68 109.6) (width 0.2) (layer "F.Cu") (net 7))
 (segment (start 199.895 112.625) (end 198.56 111.29) (width 0.2) (layer "F.Cu") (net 7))
 (segment (start 200.37 112.625) (end 199.895 112.625) (width 0.2) (layer "F.Cu") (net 7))
 (segment (start 198.56 111.29) (end 198.56 110.72) (width 0.2) (layer "F.Cu") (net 7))
 (segment (start 194.635 108.64) (end 196.87 110.875) (width 0.2) (layer "F.Cu") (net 21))
 (segment (start 191.75 108.64) (end 194.635 108.64) (width 0.2) (layer "F.Cu") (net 21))
 (segment (start 199.77 103.93) (end 198.83 104.87) (width 0.2) (layer "F.Cu") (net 24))
 (segment (start 191.2 105.54) (end 189.6 105.54) (width 0.2) (layer "F.Cu") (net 24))
 (segment (start 199.77 102.18) (end 199.77 103.93) (width 0.2) (layer "F.Cu") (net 24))
 (segment (start 189.6 105.54) (end 188.25 106.89) (width 0.2) (layer "F.Cu") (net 24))
 (via (at 198.83 104.87) (size 0.6) (drill 0.3) (layers "F.Cu" "B.Cu") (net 24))
 (via (at 191.2 105.54) (size 0.6) (drill 0.3) (layers "F.Cu" "B.Cu") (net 24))
 (segment (start 198.83 104.87) (end 191.87 104.87) (width 0.2) (layer "B.Cu") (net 24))
 (segment (start 191.87 104.87) (end 191.2 105.54) (width 0.2) (layer "B.Cu") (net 24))
 (segment (start 208.005 101.31) (end 208.82 102.125) (width 0.2) (layer "F.Cu") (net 5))
 (segment (start 197.49 99.21) (end 202.13 99.21) (width 0.2) (layer "F.Cu") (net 5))
 (segment (start 204.23 101.31) (end 208.005 101.31) (width 0.2) (layer "F.Cu") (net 5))
 (segment (start 202.13 99.21) (end 204.23 101.31) (width 0.2) (layer "F.Cu") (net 5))
 (segment (start 196.27 100.43) (end 197.49 99.21) (width 0.2) (layer "F.Cu") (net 5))
 (segment (start 215.13 94.71) (end 216.06 95.64) (width 0.2) (layer "F.Cu") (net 3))
 (segment (start 205.32 100.375) (end 210.985 94.71) (width 0.2) (layer "F.Cu") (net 3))
 (segment (start 210.985 94.71) (end 215.13 94.71) (width 0.2) (layer "F.Cu") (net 3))
 (segment (start 210.145 91.475) (end 212.56 93.89) (width 0.2) (layer "F.Cu") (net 23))
 (segment (start 206.55 91.475) (end 210.145 91.475) (width 0.2) (layer "F.Cu") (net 23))
 (segment (start 200.29 89.725) (end 196.86 93.155) (width 0.2) (layer "F.Cu") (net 22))
 (segment (start 203.05 89.725) (end 200.29 89.725) (width 0.2) (layer "F.Cu") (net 22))
 (segment (start 192.415 91.405) (end 193.36 91.405) (width 0.2) (layer "F.Cu") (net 11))
 (segment (start 188.15 95.67) (end 192.415 91.405) (width 0.2) (layer "F.Cu") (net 11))
 (segment (start 188.15 98.345) (end 188.15 95.67) (width 0.2) (layer "F.Cu") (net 11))
 (segment (start 189.93 100.125) (end 188.15 98.345) (width 0.2) (layer "F.Cu") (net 11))
 (segment (start 180.436535 140.419285) (end 184.281867 140.419285) (width 0.2) (layer "F.Cu") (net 1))
 (segment (start 198.62 140.6) (end 202.250427 140.6) (width 0.2) (layer "F.Cu") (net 1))
 (segment (start 184.281867 140.419285) (end 187.641682 143.7791) (width 0.2) (layer "F.Cu") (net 1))
 (segment (start 197.72 141.5) (end 198.62 140.6) (width 0.2) (layer "F.Cu") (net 1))
 (segment (start 199.163902 146.516069) (end 199.163902 144.213902) (width 0.2) (layer "F.Cu") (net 1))
 (segment (start 199.163902 144.213902) (end 197.72 142.77) (width 0.2) (layer "F.Cu") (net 1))
 (segment (start 197.72 142.77) (end 197.72 141.5) (width 0.2) (layer "F.Cu") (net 1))
 (segment (start 187.641682 143.7791) (end 189.978215 143.7791) (width 0.2) (layer "F.Cu") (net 1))
 (segment (start 202.250427 140.6) (end 202.646831 140.996404) (width 0.2) (layer "F.Cu") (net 1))
 (segment (start 192.220247 144.25) (end 196.897833 144.25) (width 0.2) (layer "F.Cu") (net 1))
 (segment (start 196.897833 144.25) (end 199.163902 146.516069) (width 0.2) (layer "F.Cu") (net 1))
 (segment (start 189.978215 143.7791) (end 191.334681 145.135566) (width 0.2) (layer "F.Cu") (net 1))
 (segment (start 191.334681 145.135566) (end 192.220247 144.25) (width 0.2) (layer "F.Cu") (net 1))
 (segment (start 217.667785 141.28) (end 218.096368 140.851417) (width 0.2) (layer "F.Cu") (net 12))
 (segment (start 216.19 141.28) (end 217.667785 141.28) (width 0.2) (layer "F.Cu") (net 12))
 (segment (start 190.599285 139.700715) (end 191.84 138.46) (width 0.2) (layer "F.Cu") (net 12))
 (segment (start 191.84 138.46) (end 199.96 138.46) (width 0.2) (layer "F.Cu") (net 12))
 (segment (start 189.543465 139.700715) (end 190.599285 139.700715) (width 0.2) (layer "F.Cu") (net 12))
 (segment (start 182.338318 136.3409) (end 185.698133 139.700715) (width 0.2) (layer "F.Cu") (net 12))
 (segment (start 203.42 139.69) (end 203.66 139.93) (width 0.2) (layer "F.Cu") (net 12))
 (segment (start 215.67 140.76) (end 216.19 141.28) (width 0.2) (layer "F.Cu") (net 12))
 (segment (start 199.96 138.46) (end 201.19 139.69) (width 0.2) (layer "F.Cu") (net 12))
 (segment (start 185.698133 139.700715) (end 189.543465 139.700715) (width 0.2) (layer "F.Cu") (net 12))
 (segment (start 201.19 139.69) (end 203.42 139.69) (width 0.2) (layer "F.Cu") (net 12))
 (via (at 215.67 140.76) (size 0.6) (drill 0.3) (layers "F.Cu" "B.Cu") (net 12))
 (via (at 203.66 139.93) (size 0.6) (drill 0.3) (layers "F.Cu" "B.Cu") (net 12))
 (segment (start 203.66 139.93) (end 204.01 140.28) (width 0.2) (layer "B.Cu") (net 12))
 (segment (start 215.19 140.28) (end 215.67 140.76) (width 0.2) (layer "B.Cu") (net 12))
 (segment (start 204.01 140.28) (end 214.75 140.28) (width 0.2) (layer "B.Cu") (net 12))
 (segment (start 214.75 140.28) (end 215.19 140.28) (width 0.2) (layer "B.Cu") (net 12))
 (segment (start 192.552167 141.14) (end 192.116098 140.703931) (width 0.2) (layer "F.Cu") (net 2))
 (segment (start 216.7 139.305307) (end 217.655301 138.350006) (width 0.2) (layer "F.Cu") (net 2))
 (segment (start 199.945319 142.084434) (end 198.794434 142.084434) (width 0.2) (layer "F.Cu") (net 2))
 (segment (start 198.794434 142.084434) (end 198.46 141.75) (width 0.2) (layer "F.Cu") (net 2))
 (segment (start 200.060885 142.2) (end 203.62 142.2) (width 0.2) (layer "F.Cu") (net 2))
 (segment (start 196.28 141.14) (end 192.552167 141.14) (width 0.2) (layer "F.Cu") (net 2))
 (segment (start 216.7 140.62) (end 216.7 139.305307) (width 0.2) (layer "F.Cu") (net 2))
 (segment (start 199.945319 142.084434) (end 200.060885 142.2) (width 0.2) (layer "F.Cu") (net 2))
 (via (at 198.46 141.75) (size 0.6) (drill 0.3) (layers "F.Cu" "B.Cu") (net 2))
 (via (at 203.62 142.2) (size 0.6) (drill 0.3) (layers "F.Cu" "B.Cu") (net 2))
 (via (at 216.7 140.62) (size 0.6) (drill 0.3) (layers "F.Cu" "B.Cu") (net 2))
 (via (at 196.28 141.14) (size 0.6) (drill 0.3) (layers "F.Cu" "B.Cu") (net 2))
 (segment (start 197.85 141.14) (end 196.28 141.14) (width 0.2) (layer "B.Cu") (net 2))
 (segment (start 215.12 142.2) (end 216.7 140.62) (width 0.2) (layer "B.Cu") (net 2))
 (segment (start 203.62 142.2) (end 215.12 142.2) (width 0.2) (layer "B.Cu") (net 2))
 (segment (start 198.46 141.75) (end 197.85 141.14) (width 0.2) (layer "B.Cu") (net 2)))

